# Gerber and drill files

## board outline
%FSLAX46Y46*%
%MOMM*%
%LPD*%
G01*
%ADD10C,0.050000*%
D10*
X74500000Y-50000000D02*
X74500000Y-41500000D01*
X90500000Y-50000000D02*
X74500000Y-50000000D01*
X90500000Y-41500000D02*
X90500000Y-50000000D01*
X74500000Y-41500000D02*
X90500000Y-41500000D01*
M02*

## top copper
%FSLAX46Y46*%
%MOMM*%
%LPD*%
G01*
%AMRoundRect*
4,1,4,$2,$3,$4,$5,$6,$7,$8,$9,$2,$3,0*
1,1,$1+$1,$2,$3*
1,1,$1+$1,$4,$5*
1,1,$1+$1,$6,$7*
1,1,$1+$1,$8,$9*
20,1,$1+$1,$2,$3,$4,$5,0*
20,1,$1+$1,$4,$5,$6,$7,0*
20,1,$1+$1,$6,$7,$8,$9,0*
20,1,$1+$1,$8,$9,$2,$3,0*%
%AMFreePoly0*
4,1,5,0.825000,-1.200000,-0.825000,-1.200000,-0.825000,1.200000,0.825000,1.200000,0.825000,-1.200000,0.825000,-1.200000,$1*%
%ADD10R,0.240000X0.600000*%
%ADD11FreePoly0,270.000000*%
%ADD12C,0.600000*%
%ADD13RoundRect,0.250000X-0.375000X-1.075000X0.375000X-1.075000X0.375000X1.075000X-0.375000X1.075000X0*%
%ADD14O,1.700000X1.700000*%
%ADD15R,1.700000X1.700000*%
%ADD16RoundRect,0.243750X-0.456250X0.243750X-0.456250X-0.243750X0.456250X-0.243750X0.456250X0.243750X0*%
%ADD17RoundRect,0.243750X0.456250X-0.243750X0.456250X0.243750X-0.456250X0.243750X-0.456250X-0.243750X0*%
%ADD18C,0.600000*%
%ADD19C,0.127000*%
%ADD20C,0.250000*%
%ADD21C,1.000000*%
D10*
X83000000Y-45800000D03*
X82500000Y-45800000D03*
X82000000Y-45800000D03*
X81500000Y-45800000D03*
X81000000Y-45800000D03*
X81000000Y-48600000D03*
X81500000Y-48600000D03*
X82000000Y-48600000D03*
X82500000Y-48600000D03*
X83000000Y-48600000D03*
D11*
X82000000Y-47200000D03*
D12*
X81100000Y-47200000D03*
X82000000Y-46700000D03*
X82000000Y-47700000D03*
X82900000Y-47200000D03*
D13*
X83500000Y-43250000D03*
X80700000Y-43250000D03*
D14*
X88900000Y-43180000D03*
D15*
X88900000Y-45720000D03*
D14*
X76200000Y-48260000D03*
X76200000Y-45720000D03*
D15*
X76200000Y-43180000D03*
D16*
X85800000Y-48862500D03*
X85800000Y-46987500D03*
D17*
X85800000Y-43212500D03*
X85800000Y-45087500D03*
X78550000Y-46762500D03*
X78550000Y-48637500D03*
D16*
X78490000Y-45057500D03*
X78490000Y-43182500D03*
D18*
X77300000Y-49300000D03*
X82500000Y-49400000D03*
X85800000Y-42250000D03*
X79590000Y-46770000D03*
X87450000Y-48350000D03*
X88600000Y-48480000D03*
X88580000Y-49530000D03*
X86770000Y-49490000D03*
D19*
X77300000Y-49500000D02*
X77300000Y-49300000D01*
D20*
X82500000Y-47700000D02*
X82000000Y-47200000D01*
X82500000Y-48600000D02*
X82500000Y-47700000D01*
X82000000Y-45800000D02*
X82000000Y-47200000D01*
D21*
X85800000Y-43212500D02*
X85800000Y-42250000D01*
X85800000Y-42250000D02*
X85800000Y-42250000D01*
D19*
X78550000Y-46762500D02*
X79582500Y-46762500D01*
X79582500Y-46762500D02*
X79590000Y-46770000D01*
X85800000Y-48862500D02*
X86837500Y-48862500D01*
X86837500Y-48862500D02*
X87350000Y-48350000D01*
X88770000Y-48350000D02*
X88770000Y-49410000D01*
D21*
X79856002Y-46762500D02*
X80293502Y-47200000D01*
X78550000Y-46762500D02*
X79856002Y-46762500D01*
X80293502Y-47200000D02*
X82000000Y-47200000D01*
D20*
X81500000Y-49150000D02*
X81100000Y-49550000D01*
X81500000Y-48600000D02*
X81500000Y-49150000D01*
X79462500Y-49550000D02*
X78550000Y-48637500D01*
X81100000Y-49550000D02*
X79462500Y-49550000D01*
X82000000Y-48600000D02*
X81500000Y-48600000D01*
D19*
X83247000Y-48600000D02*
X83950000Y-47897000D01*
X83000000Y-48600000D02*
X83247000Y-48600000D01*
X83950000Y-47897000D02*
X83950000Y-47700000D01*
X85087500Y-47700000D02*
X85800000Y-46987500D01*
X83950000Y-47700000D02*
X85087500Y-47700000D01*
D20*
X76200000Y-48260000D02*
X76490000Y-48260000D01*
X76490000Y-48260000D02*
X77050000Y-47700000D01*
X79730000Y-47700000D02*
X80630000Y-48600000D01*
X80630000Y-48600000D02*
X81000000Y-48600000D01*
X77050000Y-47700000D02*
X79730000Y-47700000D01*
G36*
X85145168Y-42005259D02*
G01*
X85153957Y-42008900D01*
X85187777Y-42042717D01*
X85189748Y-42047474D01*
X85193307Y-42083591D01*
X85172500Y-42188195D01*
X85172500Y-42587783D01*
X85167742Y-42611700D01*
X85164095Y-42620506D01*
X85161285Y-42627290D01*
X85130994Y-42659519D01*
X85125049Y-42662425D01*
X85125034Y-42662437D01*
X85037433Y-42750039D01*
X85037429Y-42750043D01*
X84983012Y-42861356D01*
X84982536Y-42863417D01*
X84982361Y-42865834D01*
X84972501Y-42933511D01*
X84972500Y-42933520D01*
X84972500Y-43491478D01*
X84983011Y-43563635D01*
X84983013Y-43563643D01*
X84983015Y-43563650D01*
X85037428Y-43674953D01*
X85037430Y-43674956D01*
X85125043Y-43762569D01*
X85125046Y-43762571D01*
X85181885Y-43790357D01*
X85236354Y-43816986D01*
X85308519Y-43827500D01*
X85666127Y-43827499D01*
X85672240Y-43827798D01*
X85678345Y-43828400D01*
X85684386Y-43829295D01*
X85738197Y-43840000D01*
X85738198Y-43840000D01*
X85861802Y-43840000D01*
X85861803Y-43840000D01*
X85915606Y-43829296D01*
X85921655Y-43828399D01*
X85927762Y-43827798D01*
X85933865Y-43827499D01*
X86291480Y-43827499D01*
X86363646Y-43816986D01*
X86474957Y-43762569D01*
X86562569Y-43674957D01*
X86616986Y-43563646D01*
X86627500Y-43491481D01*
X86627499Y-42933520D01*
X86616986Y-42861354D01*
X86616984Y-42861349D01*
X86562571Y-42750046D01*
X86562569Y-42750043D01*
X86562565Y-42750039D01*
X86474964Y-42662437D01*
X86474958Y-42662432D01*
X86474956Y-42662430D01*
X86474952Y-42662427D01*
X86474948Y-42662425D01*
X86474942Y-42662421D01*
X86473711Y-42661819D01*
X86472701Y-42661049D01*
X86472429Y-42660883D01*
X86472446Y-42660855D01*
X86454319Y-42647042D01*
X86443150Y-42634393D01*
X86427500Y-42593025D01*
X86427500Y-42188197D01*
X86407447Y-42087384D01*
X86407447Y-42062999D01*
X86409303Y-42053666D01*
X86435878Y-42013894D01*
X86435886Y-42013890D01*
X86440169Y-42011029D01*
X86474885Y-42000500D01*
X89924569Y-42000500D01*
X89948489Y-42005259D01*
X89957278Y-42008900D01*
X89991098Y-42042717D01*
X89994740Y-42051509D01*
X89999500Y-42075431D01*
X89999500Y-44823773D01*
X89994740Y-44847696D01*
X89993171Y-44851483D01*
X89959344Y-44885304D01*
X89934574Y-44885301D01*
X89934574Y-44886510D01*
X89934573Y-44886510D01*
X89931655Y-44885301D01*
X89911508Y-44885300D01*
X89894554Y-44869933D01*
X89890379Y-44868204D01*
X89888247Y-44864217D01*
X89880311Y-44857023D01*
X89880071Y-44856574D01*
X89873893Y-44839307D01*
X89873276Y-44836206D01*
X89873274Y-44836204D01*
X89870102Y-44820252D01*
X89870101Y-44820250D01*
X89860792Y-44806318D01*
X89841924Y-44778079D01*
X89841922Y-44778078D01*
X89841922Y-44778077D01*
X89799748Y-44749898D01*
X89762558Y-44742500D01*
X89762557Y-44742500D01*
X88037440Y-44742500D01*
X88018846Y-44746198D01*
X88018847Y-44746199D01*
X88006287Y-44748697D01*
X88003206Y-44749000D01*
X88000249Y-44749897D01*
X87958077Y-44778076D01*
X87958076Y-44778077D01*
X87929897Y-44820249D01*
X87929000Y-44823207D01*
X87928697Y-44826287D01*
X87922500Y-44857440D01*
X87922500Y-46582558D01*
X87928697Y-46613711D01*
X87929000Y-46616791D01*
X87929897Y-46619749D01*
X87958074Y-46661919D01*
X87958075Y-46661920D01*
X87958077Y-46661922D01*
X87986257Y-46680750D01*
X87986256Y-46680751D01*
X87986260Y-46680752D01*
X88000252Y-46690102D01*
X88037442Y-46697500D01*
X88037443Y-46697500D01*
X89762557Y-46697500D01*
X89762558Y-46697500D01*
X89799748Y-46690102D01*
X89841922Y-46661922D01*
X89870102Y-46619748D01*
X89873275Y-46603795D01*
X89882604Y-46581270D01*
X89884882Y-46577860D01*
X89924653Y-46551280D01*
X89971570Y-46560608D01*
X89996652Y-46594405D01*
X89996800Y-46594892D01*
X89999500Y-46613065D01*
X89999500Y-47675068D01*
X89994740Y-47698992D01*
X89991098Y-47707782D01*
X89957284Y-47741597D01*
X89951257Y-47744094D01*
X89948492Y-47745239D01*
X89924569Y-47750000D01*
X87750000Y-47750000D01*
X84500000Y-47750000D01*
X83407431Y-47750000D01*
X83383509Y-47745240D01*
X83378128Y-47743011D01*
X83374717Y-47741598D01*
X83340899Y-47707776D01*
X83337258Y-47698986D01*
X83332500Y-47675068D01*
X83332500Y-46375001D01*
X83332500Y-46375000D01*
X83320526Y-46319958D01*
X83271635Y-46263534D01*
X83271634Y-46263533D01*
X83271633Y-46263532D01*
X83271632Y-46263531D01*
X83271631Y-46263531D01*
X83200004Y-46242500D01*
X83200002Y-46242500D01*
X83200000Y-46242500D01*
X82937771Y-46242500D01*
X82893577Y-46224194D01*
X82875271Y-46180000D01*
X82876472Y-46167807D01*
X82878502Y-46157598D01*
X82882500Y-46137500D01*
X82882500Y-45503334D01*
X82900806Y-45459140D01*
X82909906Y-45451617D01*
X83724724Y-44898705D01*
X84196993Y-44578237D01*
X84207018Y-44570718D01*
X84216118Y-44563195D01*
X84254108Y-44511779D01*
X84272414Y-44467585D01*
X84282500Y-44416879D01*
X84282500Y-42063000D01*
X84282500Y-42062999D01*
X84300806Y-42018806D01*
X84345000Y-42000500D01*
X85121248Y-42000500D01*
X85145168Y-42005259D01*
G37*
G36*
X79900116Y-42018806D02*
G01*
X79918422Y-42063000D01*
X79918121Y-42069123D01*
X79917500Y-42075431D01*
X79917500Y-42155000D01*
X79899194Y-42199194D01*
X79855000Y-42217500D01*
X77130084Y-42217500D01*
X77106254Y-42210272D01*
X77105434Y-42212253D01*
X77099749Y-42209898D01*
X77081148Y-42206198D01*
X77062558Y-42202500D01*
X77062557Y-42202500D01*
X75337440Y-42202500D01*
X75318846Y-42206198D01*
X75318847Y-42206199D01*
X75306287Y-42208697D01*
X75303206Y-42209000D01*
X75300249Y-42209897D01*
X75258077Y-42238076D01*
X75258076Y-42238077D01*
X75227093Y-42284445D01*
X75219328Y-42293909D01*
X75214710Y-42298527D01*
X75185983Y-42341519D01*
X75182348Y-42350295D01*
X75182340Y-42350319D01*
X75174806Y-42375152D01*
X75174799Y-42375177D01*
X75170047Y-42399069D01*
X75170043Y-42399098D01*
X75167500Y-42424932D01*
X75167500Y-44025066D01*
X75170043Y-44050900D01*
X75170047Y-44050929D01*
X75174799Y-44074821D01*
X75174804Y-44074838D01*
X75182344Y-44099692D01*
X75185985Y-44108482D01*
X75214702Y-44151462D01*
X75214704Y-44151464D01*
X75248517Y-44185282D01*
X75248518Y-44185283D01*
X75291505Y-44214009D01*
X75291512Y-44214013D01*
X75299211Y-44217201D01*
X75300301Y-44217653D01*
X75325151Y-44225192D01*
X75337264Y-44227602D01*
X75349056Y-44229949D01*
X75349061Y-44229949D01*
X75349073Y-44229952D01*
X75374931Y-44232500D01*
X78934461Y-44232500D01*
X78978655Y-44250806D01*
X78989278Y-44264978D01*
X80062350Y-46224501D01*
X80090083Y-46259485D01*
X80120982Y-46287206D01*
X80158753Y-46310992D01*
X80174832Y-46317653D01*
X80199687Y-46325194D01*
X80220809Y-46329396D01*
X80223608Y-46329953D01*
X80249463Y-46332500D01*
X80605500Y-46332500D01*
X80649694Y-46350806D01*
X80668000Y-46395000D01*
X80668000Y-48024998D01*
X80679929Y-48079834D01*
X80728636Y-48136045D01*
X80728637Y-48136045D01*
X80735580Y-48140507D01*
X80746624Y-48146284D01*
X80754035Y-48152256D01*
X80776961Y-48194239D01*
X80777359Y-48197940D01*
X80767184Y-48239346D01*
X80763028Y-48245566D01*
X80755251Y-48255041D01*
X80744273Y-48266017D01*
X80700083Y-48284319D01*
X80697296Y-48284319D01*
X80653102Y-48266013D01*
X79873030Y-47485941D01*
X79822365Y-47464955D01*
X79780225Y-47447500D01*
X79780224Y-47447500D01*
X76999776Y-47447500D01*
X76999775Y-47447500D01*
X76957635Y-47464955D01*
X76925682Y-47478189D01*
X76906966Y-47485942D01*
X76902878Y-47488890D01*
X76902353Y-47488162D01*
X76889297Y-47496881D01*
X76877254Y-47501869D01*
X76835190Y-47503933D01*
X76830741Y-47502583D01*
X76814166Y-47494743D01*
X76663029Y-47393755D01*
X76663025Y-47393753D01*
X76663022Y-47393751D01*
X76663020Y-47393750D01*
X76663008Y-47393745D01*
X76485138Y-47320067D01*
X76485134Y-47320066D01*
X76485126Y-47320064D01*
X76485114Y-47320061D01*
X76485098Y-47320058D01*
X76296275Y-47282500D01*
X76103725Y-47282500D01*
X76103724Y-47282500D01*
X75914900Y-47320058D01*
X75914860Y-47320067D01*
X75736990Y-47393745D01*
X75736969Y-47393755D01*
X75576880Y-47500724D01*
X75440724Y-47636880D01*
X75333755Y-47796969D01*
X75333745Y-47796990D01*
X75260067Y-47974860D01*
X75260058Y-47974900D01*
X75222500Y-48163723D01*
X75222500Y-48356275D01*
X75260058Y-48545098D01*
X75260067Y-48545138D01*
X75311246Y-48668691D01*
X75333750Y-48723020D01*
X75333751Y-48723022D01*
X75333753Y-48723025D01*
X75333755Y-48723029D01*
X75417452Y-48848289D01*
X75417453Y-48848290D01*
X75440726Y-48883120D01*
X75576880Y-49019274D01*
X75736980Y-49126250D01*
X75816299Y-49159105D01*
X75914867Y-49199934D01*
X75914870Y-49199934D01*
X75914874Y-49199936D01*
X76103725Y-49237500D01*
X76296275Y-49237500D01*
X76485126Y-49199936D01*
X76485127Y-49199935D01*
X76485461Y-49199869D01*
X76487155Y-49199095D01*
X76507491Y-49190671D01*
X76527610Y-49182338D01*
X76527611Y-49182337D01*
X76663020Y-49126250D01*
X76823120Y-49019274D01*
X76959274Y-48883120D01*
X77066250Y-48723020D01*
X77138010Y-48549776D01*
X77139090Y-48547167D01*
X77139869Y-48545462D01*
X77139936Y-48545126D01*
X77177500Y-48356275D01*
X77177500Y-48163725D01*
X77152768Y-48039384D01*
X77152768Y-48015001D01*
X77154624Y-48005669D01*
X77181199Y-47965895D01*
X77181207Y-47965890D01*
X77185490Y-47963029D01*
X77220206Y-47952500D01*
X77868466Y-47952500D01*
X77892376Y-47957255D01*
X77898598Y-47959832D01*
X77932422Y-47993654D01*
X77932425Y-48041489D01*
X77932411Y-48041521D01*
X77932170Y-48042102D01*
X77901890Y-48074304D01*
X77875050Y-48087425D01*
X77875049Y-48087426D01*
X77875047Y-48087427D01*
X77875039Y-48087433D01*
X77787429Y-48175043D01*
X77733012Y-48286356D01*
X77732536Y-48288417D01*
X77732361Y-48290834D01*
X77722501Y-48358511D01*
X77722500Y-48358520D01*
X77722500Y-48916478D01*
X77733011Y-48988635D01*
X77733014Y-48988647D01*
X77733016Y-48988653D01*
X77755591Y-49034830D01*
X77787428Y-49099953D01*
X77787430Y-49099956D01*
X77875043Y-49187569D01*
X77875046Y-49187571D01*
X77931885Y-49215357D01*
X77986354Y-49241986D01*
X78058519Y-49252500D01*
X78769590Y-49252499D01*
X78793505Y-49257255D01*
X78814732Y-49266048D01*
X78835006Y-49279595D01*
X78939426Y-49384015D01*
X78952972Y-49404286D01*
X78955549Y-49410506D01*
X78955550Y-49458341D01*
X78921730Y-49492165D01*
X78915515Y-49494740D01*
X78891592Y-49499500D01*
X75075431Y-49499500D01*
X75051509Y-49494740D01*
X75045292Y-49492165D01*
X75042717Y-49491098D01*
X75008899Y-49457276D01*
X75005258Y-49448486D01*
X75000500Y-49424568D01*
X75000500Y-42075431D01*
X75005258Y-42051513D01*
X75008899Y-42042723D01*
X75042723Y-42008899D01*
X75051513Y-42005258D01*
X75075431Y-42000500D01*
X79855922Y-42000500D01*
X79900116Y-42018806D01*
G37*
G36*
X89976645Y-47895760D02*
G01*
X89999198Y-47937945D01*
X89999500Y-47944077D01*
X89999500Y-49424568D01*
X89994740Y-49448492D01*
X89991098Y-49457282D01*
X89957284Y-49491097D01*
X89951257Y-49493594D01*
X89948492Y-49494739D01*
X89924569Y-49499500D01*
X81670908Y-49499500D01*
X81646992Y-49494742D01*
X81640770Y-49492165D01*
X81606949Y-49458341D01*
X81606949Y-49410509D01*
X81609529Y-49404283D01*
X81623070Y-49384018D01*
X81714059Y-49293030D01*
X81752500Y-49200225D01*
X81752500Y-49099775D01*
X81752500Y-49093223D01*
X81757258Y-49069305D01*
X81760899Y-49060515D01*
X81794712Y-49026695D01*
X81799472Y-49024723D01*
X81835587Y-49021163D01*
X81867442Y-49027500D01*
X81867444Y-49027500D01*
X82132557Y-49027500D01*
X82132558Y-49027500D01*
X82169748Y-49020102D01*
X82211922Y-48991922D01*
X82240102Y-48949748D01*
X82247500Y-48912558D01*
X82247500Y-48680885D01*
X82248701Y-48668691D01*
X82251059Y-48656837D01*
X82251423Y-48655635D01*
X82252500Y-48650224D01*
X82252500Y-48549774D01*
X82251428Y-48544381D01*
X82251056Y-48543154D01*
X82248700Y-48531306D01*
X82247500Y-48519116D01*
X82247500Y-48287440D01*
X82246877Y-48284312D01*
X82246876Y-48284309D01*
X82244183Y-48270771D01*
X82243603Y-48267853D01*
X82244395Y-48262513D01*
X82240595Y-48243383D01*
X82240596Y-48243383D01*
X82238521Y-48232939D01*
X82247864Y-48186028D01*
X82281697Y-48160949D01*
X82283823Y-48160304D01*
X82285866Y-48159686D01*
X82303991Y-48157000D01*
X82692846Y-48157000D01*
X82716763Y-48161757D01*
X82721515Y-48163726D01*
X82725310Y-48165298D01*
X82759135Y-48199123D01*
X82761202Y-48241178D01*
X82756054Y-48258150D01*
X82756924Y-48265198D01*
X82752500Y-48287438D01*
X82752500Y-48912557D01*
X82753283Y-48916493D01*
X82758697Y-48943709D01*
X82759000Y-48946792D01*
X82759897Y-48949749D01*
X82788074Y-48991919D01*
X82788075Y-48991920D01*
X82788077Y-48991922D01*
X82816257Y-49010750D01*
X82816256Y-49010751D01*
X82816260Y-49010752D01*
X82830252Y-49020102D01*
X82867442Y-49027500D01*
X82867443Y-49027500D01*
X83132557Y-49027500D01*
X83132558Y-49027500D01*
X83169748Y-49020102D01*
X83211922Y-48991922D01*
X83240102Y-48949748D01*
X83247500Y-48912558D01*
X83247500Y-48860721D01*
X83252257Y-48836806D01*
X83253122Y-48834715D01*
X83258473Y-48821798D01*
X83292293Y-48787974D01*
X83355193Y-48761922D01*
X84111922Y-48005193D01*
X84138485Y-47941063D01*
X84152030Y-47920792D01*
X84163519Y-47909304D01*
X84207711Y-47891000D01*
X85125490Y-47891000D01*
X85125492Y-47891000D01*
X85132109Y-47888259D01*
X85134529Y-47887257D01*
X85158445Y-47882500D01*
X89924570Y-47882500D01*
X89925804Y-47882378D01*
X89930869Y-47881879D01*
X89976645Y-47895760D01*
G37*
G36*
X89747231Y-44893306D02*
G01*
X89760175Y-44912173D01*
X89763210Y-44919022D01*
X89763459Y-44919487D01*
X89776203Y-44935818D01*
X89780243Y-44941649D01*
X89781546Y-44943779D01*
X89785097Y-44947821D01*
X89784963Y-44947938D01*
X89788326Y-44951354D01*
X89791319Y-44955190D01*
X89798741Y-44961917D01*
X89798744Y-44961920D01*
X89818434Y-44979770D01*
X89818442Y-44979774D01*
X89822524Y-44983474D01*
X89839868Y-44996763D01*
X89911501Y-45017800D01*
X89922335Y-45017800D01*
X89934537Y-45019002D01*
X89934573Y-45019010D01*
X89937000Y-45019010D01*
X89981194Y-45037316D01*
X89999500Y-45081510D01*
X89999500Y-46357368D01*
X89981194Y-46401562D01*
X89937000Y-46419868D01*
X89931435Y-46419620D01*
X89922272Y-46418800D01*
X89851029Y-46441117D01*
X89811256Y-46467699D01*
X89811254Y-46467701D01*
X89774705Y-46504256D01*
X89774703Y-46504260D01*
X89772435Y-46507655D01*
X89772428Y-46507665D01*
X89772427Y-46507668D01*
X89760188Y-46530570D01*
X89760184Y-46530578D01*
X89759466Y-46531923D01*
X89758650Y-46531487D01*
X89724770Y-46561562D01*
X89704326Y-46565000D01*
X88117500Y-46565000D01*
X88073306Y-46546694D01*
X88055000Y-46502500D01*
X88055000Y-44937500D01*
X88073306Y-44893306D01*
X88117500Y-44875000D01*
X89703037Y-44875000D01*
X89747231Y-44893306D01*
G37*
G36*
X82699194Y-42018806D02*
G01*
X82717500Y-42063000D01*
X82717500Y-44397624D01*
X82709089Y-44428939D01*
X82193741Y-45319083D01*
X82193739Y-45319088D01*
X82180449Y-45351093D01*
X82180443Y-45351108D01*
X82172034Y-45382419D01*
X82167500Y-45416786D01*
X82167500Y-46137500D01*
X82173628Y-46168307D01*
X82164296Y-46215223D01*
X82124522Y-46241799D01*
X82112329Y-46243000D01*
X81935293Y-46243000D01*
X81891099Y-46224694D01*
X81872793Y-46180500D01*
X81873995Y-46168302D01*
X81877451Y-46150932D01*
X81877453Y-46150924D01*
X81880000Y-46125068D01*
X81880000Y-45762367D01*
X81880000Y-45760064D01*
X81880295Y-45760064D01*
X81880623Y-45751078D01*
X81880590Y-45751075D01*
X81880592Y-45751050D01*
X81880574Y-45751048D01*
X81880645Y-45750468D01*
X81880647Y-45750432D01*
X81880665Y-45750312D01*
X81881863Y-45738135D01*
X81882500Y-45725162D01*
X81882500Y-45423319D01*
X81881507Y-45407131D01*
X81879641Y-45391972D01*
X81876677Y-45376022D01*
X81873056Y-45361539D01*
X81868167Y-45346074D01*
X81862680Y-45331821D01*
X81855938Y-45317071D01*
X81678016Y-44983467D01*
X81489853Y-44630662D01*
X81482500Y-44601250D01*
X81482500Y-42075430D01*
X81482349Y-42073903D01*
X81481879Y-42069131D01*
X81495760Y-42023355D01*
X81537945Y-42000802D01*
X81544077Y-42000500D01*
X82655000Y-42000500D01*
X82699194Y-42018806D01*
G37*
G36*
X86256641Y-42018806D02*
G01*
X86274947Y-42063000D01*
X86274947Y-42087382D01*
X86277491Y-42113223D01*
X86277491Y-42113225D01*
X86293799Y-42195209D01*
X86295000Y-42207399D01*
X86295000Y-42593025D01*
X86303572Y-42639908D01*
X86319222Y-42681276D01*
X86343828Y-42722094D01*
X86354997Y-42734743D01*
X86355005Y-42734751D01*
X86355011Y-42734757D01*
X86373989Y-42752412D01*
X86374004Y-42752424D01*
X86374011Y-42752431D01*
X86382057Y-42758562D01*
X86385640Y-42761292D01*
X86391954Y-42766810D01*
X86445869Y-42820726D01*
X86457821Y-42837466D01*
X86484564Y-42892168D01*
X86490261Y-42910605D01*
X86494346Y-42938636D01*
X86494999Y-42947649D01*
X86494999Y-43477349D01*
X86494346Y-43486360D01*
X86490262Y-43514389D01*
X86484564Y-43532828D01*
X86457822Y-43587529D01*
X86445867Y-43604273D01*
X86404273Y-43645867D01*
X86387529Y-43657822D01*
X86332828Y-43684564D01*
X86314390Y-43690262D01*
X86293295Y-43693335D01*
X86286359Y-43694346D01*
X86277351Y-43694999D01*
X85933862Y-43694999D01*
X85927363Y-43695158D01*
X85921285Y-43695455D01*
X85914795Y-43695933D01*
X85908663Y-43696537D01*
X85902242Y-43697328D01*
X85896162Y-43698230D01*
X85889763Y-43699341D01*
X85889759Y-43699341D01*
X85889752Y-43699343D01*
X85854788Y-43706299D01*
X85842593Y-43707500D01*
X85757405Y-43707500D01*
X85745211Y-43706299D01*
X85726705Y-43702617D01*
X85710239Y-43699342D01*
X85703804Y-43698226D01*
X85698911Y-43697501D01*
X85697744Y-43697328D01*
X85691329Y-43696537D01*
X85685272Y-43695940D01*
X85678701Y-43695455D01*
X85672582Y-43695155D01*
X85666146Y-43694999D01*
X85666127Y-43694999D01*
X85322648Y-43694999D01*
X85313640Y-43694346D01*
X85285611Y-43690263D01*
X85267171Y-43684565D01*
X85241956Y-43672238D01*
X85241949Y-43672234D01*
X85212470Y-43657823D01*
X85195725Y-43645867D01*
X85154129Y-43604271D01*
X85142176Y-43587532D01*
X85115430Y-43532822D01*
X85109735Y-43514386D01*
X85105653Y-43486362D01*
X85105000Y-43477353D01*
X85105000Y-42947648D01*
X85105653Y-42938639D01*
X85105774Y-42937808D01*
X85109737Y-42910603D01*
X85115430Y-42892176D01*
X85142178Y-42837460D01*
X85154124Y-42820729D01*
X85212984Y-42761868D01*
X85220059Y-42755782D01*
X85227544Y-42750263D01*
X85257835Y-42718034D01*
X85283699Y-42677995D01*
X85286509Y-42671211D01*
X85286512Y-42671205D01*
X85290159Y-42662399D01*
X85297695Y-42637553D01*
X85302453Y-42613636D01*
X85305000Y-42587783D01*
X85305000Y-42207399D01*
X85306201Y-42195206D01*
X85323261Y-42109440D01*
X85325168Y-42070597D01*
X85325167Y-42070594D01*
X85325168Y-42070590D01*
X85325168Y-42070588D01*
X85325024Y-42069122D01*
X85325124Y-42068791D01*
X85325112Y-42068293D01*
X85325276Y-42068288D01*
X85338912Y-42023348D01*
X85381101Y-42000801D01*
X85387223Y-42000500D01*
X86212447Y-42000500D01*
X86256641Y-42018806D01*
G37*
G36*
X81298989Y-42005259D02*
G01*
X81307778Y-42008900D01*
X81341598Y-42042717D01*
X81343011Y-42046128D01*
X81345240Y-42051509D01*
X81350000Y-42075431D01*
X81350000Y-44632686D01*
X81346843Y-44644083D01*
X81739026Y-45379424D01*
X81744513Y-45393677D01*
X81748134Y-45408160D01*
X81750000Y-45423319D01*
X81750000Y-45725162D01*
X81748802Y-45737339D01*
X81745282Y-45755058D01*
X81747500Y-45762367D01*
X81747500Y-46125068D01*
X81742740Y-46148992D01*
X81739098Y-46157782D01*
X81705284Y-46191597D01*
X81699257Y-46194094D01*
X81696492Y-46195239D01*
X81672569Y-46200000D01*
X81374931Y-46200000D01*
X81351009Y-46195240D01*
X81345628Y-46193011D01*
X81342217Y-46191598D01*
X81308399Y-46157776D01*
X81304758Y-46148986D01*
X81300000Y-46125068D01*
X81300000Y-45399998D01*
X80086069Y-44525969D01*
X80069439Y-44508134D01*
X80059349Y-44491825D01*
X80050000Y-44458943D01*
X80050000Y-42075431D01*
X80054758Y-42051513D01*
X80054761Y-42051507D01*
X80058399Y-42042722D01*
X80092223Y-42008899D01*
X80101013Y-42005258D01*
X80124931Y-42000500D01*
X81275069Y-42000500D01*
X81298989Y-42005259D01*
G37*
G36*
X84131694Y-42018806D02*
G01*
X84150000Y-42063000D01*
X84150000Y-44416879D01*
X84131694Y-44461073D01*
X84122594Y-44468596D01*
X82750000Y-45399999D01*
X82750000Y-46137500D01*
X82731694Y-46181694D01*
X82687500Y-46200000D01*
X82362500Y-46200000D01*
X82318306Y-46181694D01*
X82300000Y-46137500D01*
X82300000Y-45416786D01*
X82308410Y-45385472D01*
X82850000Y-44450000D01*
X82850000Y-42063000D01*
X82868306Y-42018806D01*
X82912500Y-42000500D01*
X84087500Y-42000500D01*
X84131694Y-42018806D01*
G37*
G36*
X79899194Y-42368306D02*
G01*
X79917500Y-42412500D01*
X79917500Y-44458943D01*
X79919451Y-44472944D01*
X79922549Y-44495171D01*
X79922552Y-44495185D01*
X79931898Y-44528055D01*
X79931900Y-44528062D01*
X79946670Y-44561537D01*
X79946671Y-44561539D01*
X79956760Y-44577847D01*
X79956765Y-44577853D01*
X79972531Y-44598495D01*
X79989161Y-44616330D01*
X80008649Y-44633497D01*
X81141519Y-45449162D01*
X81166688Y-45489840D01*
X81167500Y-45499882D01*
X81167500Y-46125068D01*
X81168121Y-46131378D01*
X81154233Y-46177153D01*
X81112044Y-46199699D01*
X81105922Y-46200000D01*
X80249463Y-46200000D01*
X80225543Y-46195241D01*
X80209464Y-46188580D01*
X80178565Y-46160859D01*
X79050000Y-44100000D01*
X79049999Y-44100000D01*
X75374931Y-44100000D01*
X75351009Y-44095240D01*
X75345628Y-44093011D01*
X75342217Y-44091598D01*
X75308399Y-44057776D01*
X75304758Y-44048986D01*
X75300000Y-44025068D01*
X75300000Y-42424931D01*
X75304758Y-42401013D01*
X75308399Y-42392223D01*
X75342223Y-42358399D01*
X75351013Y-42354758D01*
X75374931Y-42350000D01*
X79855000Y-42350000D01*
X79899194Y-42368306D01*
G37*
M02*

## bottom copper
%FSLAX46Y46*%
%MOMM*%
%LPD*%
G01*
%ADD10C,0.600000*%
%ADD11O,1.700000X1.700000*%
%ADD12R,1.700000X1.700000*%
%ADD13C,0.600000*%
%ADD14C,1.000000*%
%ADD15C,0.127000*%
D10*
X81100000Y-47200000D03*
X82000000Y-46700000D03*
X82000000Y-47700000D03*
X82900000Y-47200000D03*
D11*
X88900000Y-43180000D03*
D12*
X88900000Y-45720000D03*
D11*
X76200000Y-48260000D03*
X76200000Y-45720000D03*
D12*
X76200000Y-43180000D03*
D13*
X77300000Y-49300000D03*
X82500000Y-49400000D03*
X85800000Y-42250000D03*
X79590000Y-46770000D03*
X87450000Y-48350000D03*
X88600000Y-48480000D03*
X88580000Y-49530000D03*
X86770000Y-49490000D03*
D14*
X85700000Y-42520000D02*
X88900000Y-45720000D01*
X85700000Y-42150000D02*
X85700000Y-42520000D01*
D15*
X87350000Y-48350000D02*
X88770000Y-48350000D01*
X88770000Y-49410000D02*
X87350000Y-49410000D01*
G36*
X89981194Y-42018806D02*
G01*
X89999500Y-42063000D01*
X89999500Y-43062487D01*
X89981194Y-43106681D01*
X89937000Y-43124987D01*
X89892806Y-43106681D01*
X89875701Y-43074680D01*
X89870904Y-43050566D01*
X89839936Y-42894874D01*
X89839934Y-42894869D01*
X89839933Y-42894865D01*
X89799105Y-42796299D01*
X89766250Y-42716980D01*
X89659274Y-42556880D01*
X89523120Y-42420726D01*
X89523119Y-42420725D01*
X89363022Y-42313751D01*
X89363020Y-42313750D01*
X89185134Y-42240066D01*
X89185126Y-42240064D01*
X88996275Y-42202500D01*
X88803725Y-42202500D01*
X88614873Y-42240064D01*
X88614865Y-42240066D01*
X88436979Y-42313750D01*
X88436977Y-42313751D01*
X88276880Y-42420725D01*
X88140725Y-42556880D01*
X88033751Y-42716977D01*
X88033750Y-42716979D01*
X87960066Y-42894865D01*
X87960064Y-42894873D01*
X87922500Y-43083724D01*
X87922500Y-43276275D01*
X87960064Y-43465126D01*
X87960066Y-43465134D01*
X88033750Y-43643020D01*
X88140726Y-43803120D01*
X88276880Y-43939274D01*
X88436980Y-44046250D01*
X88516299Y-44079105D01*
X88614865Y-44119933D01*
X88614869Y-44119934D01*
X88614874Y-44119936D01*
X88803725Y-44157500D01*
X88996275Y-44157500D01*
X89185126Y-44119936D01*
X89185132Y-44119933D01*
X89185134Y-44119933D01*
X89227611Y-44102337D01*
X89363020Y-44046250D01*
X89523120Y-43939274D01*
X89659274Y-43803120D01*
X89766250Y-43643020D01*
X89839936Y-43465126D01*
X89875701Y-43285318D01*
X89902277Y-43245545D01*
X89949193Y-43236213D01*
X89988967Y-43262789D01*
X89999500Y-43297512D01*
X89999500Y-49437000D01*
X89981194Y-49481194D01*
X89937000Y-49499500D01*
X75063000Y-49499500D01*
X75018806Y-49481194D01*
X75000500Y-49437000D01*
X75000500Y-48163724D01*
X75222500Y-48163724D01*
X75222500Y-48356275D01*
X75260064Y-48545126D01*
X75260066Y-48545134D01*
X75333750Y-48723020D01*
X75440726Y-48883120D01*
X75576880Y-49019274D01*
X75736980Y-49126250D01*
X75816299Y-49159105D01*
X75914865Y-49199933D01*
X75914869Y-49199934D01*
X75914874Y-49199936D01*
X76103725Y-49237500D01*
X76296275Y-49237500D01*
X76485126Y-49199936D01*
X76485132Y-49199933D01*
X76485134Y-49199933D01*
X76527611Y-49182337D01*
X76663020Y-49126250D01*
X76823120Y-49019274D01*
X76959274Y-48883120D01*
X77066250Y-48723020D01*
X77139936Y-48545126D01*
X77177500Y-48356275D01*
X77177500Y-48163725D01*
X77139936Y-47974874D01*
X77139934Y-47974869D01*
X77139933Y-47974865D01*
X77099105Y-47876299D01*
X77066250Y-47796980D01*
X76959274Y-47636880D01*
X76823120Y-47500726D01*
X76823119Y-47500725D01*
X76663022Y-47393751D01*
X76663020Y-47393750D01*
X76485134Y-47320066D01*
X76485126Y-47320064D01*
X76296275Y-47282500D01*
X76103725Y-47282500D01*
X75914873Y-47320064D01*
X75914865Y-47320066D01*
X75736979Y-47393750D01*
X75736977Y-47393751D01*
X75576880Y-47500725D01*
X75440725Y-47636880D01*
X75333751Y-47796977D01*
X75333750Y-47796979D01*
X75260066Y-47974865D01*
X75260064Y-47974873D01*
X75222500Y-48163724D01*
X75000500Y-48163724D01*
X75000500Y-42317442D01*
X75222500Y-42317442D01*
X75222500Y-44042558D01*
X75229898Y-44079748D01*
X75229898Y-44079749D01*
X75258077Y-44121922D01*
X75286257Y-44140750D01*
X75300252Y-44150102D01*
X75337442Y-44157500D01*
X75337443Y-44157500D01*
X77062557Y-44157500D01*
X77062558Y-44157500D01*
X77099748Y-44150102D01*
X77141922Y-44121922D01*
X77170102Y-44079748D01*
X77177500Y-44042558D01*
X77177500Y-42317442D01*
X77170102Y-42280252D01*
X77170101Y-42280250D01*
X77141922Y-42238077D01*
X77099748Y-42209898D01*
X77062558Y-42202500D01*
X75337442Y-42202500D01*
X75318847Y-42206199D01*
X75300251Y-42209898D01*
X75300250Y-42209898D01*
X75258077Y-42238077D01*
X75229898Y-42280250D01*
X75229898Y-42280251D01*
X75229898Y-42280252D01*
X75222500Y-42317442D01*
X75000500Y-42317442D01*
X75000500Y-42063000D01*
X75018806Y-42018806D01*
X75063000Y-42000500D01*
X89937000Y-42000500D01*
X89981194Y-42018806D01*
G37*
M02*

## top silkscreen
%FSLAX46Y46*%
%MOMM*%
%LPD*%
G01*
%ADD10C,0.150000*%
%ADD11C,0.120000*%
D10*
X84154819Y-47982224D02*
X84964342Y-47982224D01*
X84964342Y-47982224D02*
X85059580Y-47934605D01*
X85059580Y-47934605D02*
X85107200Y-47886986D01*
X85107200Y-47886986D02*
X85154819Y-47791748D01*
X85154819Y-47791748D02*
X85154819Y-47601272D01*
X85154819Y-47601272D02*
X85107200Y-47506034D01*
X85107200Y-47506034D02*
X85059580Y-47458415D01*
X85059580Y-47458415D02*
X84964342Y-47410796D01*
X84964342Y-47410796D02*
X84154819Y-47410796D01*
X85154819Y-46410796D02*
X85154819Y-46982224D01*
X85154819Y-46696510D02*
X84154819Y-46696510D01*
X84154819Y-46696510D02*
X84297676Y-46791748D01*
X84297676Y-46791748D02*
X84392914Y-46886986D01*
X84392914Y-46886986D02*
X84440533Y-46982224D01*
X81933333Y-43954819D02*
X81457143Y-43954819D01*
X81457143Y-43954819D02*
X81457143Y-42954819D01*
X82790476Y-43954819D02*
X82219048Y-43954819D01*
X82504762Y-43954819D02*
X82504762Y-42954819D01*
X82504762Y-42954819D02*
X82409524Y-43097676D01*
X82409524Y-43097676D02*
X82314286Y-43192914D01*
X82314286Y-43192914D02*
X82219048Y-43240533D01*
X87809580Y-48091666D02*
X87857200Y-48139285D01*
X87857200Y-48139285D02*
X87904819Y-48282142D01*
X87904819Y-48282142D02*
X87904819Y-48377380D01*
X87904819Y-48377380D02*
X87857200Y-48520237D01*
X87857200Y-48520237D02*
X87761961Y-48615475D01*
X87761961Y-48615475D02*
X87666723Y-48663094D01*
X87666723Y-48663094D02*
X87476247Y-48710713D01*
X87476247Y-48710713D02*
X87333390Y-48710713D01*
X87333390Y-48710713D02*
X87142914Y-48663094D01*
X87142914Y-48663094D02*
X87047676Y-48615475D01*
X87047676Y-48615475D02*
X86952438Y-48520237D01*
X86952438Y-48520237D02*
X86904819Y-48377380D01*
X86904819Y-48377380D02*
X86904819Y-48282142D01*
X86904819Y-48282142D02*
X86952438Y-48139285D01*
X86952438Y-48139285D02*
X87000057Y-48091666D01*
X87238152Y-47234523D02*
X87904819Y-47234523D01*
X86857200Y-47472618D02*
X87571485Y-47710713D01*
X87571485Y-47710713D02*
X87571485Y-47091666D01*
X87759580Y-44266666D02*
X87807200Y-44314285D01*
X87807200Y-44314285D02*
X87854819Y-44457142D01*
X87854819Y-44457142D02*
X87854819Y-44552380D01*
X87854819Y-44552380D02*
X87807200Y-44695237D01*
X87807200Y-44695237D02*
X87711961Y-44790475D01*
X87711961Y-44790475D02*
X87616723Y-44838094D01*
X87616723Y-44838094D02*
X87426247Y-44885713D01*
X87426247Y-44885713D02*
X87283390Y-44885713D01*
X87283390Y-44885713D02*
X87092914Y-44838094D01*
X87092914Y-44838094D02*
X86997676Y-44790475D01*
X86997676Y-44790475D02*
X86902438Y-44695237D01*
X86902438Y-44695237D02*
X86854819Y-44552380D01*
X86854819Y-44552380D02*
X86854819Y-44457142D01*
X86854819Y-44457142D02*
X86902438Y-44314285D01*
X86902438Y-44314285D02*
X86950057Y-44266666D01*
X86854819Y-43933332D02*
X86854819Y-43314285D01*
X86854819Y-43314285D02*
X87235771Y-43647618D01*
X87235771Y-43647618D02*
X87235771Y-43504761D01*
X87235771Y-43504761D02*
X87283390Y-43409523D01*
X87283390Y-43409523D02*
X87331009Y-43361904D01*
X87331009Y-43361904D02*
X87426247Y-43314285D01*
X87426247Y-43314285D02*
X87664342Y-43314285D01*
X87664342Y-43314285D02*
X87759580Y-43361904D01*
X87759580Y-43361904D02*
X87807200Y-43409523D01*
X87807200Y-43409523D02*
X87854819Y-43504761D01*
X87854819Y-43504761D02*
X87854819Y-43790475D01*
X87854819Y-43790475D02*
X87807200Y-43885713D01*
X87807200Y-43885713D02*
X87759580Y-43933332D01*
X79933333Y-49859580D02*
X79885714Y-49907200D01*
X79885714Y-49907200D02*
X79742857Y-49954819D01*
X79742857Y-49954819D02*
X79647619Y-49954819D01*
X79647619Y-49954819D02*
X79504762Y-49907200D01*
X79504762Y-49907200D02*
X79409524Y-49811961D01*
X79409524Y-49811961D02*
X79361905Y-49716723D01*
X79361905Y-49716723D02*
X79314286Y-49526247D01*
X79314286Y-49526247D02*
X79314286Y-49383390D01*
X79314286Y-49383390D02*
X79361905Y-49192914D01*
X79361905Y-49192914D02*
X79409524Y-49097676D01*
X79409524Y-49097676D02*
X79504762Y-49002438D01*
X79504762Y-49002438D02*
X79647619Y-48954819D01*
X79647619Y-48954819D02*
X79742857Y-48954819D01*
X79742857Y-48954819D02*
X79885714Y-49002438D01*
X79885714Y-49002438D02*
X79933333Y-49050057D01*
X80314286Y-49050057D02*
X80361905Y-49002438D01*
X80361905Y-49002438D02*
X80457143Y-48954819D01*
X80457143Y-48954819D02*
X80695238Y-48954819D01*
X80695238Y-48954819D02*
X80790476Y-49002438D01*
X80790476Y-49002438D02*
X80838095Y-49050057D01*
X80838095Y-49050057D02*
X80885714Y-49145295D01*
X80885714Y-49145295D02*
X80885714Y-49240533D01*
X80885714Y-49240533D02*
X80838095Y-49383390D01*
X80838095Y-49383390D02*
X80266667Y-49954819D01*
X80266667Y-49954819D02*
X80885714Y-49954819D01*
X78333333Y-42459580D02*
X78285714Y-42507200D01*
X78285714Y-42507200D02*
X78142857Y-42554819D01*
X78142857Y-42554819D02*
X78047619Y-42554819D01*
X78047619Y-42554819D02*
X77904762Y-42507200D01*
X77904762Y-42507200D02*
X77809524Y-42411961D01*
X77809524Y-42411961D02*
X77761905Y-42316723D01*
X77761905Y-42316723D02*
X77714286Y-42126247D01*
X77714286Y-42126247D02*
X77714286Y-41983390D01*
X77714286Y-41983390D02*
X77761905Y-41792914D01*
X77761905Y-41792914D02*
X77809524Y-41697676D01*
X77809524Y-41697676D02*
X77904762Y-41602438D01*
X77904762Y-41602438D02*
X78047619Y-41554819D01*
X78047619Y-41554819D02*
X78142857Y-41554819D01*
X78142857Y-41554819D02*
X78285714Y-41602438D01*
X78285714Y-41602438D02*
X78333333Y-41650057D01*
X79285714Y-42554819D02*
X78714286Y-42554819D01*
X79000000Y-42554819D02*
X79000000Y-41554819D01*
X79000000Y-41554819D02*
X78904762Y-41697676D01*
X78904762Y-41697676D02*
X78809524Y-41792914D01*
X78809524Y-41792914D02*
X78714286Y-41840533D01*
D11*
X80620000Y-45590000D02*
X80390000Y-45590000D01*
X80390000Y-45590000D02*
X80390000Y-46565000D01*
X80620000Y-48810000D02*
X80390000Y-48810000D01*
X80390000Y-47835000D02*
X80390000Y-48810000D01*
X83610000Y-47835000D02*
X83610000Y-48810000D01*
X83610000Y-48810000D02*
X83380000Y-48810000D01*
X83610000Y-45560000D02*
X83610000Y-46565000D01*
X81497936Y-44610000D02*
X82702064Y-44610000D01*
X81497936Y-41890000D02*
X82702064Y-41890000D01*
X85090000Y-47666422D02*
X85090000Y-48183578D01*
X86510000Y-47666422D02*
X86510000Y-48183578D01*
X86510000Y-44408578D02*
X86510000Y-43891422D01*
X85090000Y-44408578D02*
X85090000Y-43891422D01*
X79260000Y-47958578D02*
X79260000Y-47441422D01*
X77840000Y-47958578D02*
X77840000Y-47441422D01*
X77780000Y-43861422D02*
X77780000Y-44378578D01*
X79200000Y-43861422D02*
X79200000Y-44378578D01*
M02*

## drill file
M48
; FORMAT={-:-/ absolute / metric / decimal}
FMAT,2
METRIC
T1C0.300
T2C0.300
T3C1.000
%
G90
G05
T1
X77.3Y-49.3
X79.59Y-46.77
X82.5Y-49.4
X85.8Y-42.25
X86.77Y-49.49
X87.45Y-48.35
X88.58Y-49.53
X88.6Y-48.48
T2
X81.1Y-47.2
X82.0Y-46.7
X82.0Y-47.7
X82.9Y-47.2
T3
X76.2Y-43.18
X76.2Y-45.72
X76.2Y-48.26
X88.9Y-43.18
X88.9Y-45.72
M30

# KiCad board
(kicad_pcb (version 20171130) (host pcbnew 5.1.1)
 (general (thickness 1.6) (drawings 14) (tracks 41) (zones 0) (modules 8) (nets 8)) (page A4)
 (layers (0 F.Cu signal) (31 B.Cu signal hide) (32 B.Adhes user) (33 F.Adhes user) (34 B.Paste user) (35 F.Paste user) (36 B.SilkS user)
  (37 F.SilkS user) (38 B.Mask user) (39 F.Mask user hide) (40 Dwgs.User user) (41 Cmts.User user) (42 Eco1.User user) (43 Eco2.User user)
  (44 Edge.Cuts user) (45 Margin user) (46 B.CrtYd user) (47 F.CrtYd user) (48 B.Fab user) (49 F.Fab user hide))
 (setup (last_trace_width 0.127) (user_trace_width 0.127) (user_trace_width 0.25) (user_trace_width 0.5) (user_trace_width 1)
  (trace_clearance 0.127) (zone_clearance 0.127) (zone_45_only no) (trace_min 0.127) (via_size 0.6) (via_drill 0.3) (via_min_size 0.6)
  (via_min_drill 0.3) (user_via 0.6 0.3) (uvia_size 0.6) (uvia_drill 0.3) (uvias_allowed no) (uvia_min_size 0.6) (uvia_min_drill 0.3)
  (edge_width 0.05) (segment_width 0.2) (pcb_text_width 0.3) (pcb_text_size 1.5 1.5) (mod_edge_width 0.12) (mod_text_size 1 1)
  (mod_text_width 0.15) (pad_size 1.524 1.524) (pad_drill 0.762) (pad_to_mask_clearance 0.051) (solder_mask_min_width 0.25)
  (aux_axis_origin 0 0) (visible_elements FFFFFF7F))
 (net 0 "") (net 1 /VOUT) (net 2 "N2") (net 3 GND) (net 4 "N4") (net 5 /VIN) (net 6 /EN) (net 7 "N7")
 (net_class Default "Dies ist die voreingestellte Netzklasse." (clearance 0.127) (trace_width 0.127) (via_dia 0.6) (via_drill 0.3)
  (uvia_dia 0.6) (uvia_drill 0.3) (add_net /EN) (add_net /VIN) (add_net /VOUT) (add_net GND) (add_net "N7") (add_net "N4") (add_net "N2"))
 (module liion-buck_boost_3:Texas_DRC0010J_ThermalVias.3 (layer F.Cu) (at 82 47.2 270)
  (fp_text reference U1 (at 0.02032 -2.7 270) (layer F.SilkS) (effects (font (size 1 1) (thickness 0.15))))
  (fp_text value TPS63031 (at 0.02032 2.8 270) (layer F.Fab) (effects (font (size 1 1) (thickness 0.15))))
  (fp_line (start -1.61 1.38) (end -1.61 1.61) (layer F.SilkS) (width 0.12))
  (fp_line (start -1.61 1.61) (end -0.635 1.61) (layer F.SilkS) (width 0.12))
  (fp_line (start 1.61 1.38) (end 1.61 1.61) (layer F.SilkS) (width 0.12))
  (fp_line (start 0.635 1.61) (end 1.61 1.61) (layer F.SilkS) (width 0.12))
  (fp_line (start 0.635 -1.61) (end 1.61 -1.61) (layer F.SilkS) (width 0.12))
  (fp_line (start 1.61 -1.61) (end 1.61 -1.38) (layer F.SilkS) (width 0.12))
  (fp_line (start -1.64 -1.61) (end -0.635 -1.61) (layer F.SilkS) (width 0.12))
  (pad "" smd roundrect (at 0 0.63 270) (size 1.5 1.06) (layers F.Paste) (roundrect_rratio 0.1) (zone_connect 0))
  (pad "" smd roundrect (at 0 -0.63 270) (size 1.5 1.06) (layers F.Paste) (roundrect_rratio 0.1) (zone_connect 0))
  (pad "" smd roundrect (at -0.25 -1.53 270) (size 0.25 0.34) (layers F.Paste) (roundrect_rratio 0.1) (zone_connect 0))
  (pad "" smd roundrect (at 0.25 -1.53 270) (size 0.25 0.34) (layers F.Paste) (roundrect_rratio 0.1) (zone_connect 0))
  (pad "" smd roundrect (at -0.25 1.53 270) (size 0.25 0.34) (layers F.Paste) (roundrect_rratio 0.1) (zone_connect 0))
  (pad "" smd roundrect (at 0.25 1.53 270) (size 0.25 0.34) (layers F.Paste) (roundrect_rratio 0.1) (zone_connect 0))
  (pad 1 smd rect (at -1.4 -1 270) (size 0.6 0.24) (layers F.Cu F.Paste F.Mask) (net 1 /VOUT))
  (pad 2 smd rect (at -1.4 -0.5 270) (size 0.6 0.24) (layers F.Cu F.Paste F.Mask) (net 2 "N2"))
  (pad 3 smd rect (at -1.4 0 270) (size 0.6 0.24) (layers F.Cu F.Paste F.Mask) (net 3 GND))
  (pad 4 smd rect (at -1.4 0.5 270) (size 0.6 0.24) (layers F.Cu F.Paste F.Mask) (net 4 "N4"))
  (pad 5 smd rect (at -1.4 1 270) (size 0.6 0.24) (layers F.Cu F.Paste F.Mask) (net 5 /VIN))
  (pad 6 smd rect (at 1.4 1 270) (size 0.6 0.24) (layers F.Cu F.Paste F.Mask) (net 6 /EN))
  (pad 7 smd rect (at 1.4 0.5 270) (size 0.6 0.24) (layers F.Cu F.Paste F.Mask) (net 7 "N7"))
  (pad 8 smd rect (at 1.4 0 270) (size 0.6 0.24) (layers F.Cu F.Paste F.Mask) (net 7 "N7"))
  (pad 9 smd rect (at 1.4 -0.5 270) (size 0.6 0.24) (layers F.Cu F.Paste F.Mask) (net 3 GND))
  (pad 10 smd rect (at 1.4 -1 270) (size 0.6 0.24) (layers F.Cu F.Paste F.Mask) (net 1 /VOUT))
  (pad 11 smd custom (at 0 0 270) (size 1.65 2.4) (layers F.Cu F.Mask) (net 3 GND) (zone_connect 0)
   (options (clearance outline) (anchor rect)) (primitives))
  (pad 11 thru_hole circle (at 0 0.9 270) (size 0.6 0.6) (drill 0.3) (layers *.Cu) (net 3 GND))
  (pad 11 thru_hole circle (at -0.5 0 270) (size 0.6 0.6) (drill 0.3) (layers *.Cu) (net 3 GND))
  (pad 11 thru_hole circle (at 0.5 0 270) (size 0.6 0.6) (drill 0.3) (layers *.Cu) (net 3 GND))
  (pad 11 thru_hole circle (at 0 -0.9 270) (size 0.6 0.6) (drill 0.3) (layers *.Cu) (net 3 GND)))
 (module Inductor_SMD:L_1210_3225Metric (layer F.Cu) (at 82.1 43.25)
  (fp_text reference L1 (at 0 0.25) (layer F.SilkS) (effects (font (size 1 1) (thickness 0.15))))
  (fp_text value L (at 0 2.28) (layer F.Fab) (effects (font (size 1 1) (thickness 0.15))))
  (fp_line (start -0.602064 1.36) (end 0.602064 1.36) (layer F.SilkS) (width 0.12))
  (fp_line (start -0.602064 -1.36) (end 0.602064 -1.36) (layer F.SilkS) (width 0.12))
  (pad 2 smd roundrect (at 1.4 0) (size 1.25 2.65) (layers F.Cu F.Paste F.Mask) (roundrect_rratio 0.2) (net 2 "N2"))
  (pad 1 smd roundrect (at -1.4 0) (size 1.25 2.65) (layers F.Cu F.Paste F.Mask) (roundrect_rratio 0.2) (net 4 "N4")))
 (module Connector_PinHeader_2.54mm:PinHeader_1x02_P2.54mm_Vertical (layer B.Cu) (at 88.9 45.72)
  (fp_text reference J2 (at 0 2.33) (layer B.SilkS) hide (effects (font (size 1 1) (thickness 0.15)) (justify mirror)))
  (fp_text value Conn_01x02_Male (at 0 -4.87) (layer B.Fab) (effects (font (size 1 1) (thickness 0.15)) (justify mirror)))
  (pad 2 thru_hole oval (at 0 -2.54) (size 1.7 1.7) (drill 1) (layers *.Cu *.Mask) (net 1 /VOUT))
  (pad 1 thru_hole rect (at 0 0) (size 1.7 1.7) (drill 1) (layers *.Cu *.Mask) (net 3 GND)))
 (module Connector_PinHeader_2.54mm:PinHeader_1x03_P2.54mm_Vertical (layer B.Cu) (at 76.2 43.18 180)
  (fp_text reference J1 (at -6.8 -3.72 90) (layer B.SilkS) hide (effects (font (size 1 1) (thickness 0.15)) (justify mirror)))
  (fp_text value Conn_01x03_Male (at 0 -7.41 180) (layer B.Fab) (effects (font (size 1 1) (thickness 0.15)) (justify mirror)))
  (pad 3 thru_hole oval (at 0 -5.08 180) (size 1.7 1.7) (drill 1) (layers *.Cu *.Mask) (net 6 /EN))
  (pad 2 thru_hole oval (at 0 -2.54 180) (size 1.7 1.7) (drill 1) (layers *.Cu *.Mask) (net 3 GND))
  (pad 1 thru_hole rect (at 0 0 180) (size 1.7 1.7) (drill 1) (layers *.Cu *.Mask) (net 5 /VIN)))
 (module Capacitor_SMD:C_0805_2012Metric (layer F.Cu) (at 85.8 47.925 270)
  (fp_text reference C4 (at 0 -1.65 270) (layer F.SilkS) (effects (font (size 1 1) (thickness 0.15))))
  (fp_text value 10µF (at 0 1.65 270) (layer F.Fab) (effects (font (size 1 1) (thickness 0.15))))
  (fp_line (start -0.258578 0.71) (end 0.258578 0.71) (layer F.SilkS) (width 0.12))
  (fp_line (start -0.258578 -0.71) (end 0.258578 -0.71) (layer F.SilkS) (width 0.12))
  (pad 2 smd roundrect (at 0.9375 0 270) (size 0.975 1.4) (layers F.Cu F.Paste F.Mask) (roundrect_rratio 0.25) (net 3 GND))
  (pad 1 smd roundrect (at -0.9375 0 270) (size 0.975 1.4) (layers F.Cu F.Paste F.Mask) (roundrect_rratio 0.25) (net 1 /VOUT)))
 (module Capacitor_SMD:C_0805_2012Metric (layer F.Cu) (at 85.8 44.15 90)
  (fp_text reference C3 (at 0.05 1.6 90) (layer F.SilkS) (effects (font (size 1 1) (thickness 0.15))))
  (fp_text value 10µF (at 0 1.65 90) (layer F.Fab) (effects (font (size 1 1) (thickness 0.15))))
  (fp_line (start -0.258578 0.71) (end 0.258578 0.71) (layer F.SilkS) (width 0.12))
  (fp_line (start -0.258578 -0.71) (end 0.258578 -0.71) (layer F.SilkS) (width 0.12))
  (pad 2 smd roundrect (at 0.9375 0 90) (size 0.975 1.4) (layers F.Cu F.Paste F.Mask) (roundrect_rratio 0.25) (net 3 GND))
  (pad 1 smd roundrect (at -0.9375 0 90) (size 0.975 1.4) (layers F.Cu F.Paste F.Mask) (roundrect_rratio 0.25) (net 1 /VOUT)))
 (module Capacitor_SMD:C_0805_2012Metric (layer F.Cu) (at 78.55 47.7 90)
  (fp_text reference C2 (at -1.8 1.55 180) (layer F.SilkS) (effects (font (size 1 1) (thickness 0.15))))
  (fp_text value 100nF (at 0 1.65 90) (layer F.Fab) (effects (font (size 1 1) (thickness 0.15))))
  (fp_line (start -0.258578 0.71) (end 0.258578 0.71) (layer F.SilkS) (width 0.12))
  (fp_line (start -0.258578 -0.71) (end 0.258578 -0.71) (layer F.SilkS) (width 0.12))
  (pad 2 smd roundrect (at 0.9375 0 90) (size 0.975 1.4) (layers F.Cu F.Paste F.Mask) (roundrect_rratio 0.25) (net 3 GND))
  (pad 1 smd roundrect (at -0.9375 0 90) (size 0.975 1.4) (layers F.Cu F.Paste F.Mask) (roundrect_rratio 0.25) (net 7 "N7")))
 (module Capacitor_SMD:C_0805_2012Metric (layer F.Cu) (at 78.49 44.12 270)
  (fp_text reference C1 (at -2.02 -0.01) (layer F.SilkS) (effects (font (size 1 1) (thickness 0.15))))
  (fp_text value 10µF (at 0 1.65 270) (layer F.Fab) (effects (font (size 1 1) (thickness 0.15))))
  (fp_line (start -0.258578 0.71) (end 0.258578 0.71) (layer F.SilkS) (width 0.12))
  (fp_line (start -0.258578 -0.71) (end 0.258578 -0.71) (layer F.SilkS) (width 0.12))
  (pad 2 smd roundrect (at 0.9375 0 270) (size 0.975 1.4) (layers F.Cu F.Paste F.Mask) (roundrect_rratio 0.25) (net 3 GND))
  (pad 1 smd roundrect (at -0.9375 0 270) (size 0.975 1.4) (layers F.Cu F.Paste F.Mask) (roundrect_rratio 0.25) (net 5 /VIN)))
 (gr_line (start 74.5 50) (end 74.5 41.5) (layer Edge.Cuts) (width 0.05))
 (gr_line (start 90.5 50) (end 74.5 50) (layer Edge.Cuts) (width 0.05))
 (gr_line (start 90.5 41.5) (end 90.5 50) (layer Edge.Cuts) (width 0.05))
 (gr_line (start 74.5 41.5) (end 90.5 41.5) (layer Edge.Cuts) (width 0.05))
 (via (at 77.3 49.3) (size 0.6) (drill 0.3) (layers F.Cu B.Cu) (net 3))
 (segment (start 77.3 49.5) (end 77.3 49.3) (width 0.127) (layer F.Cu) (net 3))
 (via (at 82.5 49.4) (size 0.6) (drill 0.3) (layers F.Cu B.Cu) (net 3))
 (segment (start 82.5 47.7) (end 82 47.2) (width 0.25) (layer F.Cu) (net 3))
 (segment (start 82.5 48.6) (end 82.5 47.7) (width 0.25) (layer F.Cu) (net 3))
 (segment (start 82 45.8) (end 82 47.2) (width 0.25) (layer F.Cu) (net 3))
 (segment (start 85.8 43.2125) (end 85.8 42.25) (width 1) (layer F.Cu) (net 3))
 (segment (start 85.7 42.52) (end 88.9 45.72) (width 1) (layer B.Cu) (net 3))
 (segment (start 85.7 42.15) (end 85.7 42.52) (width 1) (layer B.Cu) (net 3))
 (segment (start 85.8 42.25) (end 85.8 42.25) (width 1) (layer F.Cu) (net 3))
 (via (at 85.8 42.25) (size 0.6) (drill 0.3) (layers F.Cu B.Cu) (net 3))
 (segment (start 78.55 46.7625) (end 79.5825 46.7625) (width 0.127) (layer F.Cu) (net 3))
 (via (at 79.59 46.77) (size 0.6) (drill 0.3) (layers F.Cu B.Cu) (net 3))
 (segment (start 79.5825 46.7625) (end 79.59 46.77) (width 0.127) (layer F.Cu) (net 3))
 (segment (start 85.8 48.8625) (end 86.8375 48.8625) (width 0.127) (layer F.Cu) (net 3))
 (via (at 87.45 48.35) (size 0.6) (drill 0.3) (layers F.Cu B.Cu) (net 3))
 (segment (start 86.8375 48.8625) (end 87.35 48.35) (width 0.127) (layer F.Cu) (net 3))
 (via (at 88.6 48.48) (size 0.6) (drill 0.3) (layers F.Cu B.Cu) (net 3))
 (segment (start 87.35 48.35) (end 88.77 48.35) (width 0.127) (layer B.Cu) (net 3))
 (via (at 88.58 49.53) (size 0.6) (drill 0.3) (layers F.Cu B.Cu) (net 3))
 (segment (start 88.77 48.35) (end 88.77 49.41) (width 0.127) (layer F.Cu) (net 3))
 (via (at 86.77 49.49) (size 0.6) (drill 0.3) (layers F.Cu B.Cu) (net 3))
 (segment (start 88.77 49.41) (end 87.35 49.41) (width 0.127) (layer B.Cu) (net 3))
 (segment (start 79.856002 46.7625) (end 80.293502 47.2) (width 1) (layer F.Cu) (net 3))
 (segment (start 78.55 46.7625) (end 79.856002 46.7625) (width 1) (layer F.Cu) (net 3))
 (segment (start 80.293502 47.2) (end 82 47.2) (width 1) (layer F.Cu) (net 3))
 (segment (start 81.5 49.15) (end 81.1 49.55) (width 0.25) (layer F.Cu) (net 7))
 (segment (start 81.5 48.6) (end 81.5 49.15) (width 0.25) (layer F.Cu) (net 7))
 (segment (start 79.4625 49.55) (end 78.55 48.6375) (width 0.25) (layer F.Cu) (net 7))
 (segment (start 81.1 49.55) (end 79.4625 49.55) (width 0.25) (layer F.Cu) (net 7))
 (segment (start 82 48.6) (end 81.5 48.6) (width 0.25) (layer F.Cu) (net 7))
 (segment (start 83.247 48.6) (end 83.95 47.897) (width 0.127) (layer F.Cu) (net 1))
 (segment (start 83 48.6) (end 83.247 48.6) (width 0.127) (layer F.Cu) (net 1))
 (segment (start 83.95 47.897) (end 83.95 47.7) (width 0.127) (layer F.Cu) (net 1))
 (segment (start 85.0875 47.7) (end 85.8 46.9875) (width 0.127) (layer F.Cu) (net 1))
 (segment (start 83.95 47.7) (end 85.0875 47.7) (width 0.127) (layer F.Cu) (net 1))
 (segment (start 76.2 48.26) (end 76.49 48.26) (width 0.25) (layer F.Cu) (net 6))
 (segment (start 76.49 48.26) (end 77.05 47.7) (width 0.25) (layer F.Cu) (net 6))
 (segment (start 79.73 47.7) (end 80.63 48.6) (width 0.25) (layer F.Cu) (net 6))
 (segment (start 80.63 48.6) (end 81 48.6) (width 0.25) (layer F.Cu) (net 6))
 (segment (start 77.05 47.7) (end 79.73 47.7) (width 0.25) (layer F.Cu) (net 6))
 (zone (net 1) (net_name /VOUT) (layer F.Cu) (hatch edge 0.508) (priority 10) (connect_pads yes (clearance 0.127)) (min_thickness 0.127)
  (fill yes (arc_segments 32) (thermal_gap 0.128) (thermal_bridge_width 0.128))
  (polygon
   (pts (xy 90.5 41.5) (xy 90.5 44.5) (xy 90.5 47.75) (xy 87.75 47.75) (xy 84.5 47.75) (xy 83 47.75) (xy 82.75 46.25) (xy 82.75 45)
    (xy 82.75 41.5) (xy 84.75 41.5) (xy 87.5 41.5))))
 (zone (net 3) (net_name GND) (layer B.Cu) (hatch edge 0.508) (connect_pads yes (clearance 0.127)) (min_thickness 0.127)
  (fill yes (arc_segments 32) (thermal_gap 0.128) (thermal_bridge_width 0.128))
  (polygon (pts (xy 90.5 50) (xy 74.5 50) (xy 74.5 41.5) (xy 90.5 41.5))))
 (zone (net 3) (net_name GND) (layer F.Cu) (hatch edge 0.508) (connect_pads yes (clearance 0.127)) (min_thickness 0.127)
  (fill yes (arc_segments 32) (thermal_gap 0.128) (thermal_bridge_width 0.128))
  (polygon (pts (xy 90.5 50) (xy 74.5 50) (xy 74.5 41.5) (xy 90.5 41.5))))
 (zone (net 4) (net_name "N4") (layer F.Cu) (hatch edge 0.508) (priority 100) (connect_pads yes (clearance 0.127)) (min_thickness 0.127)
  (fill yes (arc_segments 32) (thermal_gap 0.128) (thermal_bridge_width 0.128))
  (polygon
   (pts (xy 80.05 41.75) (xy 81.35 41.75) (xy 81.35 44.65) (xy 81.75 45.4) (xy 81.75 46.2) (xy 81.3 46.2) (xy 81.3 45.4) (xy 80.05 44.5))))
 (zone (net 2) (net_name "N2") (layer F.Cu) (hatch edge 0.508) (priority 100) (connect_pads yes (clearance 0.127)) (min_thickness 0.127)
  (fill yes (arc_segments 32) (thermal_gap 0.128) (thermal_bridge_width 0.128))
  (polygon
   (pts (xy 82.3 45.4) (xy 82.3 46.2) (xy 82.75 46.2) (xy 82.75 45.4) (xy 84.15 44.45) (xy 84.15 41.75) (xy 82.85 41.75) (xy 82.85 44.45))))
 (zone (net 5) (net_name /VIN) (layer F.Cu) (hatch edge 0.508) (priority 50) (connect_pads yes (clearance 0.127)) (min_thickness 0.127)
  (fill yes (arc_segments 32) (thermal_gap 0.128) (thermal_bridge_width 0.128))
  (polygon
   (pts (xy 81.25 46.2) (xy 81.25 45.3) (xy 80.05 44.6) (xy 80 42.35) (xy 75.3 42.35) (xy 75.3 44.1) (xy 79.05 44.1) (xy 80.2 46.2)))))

